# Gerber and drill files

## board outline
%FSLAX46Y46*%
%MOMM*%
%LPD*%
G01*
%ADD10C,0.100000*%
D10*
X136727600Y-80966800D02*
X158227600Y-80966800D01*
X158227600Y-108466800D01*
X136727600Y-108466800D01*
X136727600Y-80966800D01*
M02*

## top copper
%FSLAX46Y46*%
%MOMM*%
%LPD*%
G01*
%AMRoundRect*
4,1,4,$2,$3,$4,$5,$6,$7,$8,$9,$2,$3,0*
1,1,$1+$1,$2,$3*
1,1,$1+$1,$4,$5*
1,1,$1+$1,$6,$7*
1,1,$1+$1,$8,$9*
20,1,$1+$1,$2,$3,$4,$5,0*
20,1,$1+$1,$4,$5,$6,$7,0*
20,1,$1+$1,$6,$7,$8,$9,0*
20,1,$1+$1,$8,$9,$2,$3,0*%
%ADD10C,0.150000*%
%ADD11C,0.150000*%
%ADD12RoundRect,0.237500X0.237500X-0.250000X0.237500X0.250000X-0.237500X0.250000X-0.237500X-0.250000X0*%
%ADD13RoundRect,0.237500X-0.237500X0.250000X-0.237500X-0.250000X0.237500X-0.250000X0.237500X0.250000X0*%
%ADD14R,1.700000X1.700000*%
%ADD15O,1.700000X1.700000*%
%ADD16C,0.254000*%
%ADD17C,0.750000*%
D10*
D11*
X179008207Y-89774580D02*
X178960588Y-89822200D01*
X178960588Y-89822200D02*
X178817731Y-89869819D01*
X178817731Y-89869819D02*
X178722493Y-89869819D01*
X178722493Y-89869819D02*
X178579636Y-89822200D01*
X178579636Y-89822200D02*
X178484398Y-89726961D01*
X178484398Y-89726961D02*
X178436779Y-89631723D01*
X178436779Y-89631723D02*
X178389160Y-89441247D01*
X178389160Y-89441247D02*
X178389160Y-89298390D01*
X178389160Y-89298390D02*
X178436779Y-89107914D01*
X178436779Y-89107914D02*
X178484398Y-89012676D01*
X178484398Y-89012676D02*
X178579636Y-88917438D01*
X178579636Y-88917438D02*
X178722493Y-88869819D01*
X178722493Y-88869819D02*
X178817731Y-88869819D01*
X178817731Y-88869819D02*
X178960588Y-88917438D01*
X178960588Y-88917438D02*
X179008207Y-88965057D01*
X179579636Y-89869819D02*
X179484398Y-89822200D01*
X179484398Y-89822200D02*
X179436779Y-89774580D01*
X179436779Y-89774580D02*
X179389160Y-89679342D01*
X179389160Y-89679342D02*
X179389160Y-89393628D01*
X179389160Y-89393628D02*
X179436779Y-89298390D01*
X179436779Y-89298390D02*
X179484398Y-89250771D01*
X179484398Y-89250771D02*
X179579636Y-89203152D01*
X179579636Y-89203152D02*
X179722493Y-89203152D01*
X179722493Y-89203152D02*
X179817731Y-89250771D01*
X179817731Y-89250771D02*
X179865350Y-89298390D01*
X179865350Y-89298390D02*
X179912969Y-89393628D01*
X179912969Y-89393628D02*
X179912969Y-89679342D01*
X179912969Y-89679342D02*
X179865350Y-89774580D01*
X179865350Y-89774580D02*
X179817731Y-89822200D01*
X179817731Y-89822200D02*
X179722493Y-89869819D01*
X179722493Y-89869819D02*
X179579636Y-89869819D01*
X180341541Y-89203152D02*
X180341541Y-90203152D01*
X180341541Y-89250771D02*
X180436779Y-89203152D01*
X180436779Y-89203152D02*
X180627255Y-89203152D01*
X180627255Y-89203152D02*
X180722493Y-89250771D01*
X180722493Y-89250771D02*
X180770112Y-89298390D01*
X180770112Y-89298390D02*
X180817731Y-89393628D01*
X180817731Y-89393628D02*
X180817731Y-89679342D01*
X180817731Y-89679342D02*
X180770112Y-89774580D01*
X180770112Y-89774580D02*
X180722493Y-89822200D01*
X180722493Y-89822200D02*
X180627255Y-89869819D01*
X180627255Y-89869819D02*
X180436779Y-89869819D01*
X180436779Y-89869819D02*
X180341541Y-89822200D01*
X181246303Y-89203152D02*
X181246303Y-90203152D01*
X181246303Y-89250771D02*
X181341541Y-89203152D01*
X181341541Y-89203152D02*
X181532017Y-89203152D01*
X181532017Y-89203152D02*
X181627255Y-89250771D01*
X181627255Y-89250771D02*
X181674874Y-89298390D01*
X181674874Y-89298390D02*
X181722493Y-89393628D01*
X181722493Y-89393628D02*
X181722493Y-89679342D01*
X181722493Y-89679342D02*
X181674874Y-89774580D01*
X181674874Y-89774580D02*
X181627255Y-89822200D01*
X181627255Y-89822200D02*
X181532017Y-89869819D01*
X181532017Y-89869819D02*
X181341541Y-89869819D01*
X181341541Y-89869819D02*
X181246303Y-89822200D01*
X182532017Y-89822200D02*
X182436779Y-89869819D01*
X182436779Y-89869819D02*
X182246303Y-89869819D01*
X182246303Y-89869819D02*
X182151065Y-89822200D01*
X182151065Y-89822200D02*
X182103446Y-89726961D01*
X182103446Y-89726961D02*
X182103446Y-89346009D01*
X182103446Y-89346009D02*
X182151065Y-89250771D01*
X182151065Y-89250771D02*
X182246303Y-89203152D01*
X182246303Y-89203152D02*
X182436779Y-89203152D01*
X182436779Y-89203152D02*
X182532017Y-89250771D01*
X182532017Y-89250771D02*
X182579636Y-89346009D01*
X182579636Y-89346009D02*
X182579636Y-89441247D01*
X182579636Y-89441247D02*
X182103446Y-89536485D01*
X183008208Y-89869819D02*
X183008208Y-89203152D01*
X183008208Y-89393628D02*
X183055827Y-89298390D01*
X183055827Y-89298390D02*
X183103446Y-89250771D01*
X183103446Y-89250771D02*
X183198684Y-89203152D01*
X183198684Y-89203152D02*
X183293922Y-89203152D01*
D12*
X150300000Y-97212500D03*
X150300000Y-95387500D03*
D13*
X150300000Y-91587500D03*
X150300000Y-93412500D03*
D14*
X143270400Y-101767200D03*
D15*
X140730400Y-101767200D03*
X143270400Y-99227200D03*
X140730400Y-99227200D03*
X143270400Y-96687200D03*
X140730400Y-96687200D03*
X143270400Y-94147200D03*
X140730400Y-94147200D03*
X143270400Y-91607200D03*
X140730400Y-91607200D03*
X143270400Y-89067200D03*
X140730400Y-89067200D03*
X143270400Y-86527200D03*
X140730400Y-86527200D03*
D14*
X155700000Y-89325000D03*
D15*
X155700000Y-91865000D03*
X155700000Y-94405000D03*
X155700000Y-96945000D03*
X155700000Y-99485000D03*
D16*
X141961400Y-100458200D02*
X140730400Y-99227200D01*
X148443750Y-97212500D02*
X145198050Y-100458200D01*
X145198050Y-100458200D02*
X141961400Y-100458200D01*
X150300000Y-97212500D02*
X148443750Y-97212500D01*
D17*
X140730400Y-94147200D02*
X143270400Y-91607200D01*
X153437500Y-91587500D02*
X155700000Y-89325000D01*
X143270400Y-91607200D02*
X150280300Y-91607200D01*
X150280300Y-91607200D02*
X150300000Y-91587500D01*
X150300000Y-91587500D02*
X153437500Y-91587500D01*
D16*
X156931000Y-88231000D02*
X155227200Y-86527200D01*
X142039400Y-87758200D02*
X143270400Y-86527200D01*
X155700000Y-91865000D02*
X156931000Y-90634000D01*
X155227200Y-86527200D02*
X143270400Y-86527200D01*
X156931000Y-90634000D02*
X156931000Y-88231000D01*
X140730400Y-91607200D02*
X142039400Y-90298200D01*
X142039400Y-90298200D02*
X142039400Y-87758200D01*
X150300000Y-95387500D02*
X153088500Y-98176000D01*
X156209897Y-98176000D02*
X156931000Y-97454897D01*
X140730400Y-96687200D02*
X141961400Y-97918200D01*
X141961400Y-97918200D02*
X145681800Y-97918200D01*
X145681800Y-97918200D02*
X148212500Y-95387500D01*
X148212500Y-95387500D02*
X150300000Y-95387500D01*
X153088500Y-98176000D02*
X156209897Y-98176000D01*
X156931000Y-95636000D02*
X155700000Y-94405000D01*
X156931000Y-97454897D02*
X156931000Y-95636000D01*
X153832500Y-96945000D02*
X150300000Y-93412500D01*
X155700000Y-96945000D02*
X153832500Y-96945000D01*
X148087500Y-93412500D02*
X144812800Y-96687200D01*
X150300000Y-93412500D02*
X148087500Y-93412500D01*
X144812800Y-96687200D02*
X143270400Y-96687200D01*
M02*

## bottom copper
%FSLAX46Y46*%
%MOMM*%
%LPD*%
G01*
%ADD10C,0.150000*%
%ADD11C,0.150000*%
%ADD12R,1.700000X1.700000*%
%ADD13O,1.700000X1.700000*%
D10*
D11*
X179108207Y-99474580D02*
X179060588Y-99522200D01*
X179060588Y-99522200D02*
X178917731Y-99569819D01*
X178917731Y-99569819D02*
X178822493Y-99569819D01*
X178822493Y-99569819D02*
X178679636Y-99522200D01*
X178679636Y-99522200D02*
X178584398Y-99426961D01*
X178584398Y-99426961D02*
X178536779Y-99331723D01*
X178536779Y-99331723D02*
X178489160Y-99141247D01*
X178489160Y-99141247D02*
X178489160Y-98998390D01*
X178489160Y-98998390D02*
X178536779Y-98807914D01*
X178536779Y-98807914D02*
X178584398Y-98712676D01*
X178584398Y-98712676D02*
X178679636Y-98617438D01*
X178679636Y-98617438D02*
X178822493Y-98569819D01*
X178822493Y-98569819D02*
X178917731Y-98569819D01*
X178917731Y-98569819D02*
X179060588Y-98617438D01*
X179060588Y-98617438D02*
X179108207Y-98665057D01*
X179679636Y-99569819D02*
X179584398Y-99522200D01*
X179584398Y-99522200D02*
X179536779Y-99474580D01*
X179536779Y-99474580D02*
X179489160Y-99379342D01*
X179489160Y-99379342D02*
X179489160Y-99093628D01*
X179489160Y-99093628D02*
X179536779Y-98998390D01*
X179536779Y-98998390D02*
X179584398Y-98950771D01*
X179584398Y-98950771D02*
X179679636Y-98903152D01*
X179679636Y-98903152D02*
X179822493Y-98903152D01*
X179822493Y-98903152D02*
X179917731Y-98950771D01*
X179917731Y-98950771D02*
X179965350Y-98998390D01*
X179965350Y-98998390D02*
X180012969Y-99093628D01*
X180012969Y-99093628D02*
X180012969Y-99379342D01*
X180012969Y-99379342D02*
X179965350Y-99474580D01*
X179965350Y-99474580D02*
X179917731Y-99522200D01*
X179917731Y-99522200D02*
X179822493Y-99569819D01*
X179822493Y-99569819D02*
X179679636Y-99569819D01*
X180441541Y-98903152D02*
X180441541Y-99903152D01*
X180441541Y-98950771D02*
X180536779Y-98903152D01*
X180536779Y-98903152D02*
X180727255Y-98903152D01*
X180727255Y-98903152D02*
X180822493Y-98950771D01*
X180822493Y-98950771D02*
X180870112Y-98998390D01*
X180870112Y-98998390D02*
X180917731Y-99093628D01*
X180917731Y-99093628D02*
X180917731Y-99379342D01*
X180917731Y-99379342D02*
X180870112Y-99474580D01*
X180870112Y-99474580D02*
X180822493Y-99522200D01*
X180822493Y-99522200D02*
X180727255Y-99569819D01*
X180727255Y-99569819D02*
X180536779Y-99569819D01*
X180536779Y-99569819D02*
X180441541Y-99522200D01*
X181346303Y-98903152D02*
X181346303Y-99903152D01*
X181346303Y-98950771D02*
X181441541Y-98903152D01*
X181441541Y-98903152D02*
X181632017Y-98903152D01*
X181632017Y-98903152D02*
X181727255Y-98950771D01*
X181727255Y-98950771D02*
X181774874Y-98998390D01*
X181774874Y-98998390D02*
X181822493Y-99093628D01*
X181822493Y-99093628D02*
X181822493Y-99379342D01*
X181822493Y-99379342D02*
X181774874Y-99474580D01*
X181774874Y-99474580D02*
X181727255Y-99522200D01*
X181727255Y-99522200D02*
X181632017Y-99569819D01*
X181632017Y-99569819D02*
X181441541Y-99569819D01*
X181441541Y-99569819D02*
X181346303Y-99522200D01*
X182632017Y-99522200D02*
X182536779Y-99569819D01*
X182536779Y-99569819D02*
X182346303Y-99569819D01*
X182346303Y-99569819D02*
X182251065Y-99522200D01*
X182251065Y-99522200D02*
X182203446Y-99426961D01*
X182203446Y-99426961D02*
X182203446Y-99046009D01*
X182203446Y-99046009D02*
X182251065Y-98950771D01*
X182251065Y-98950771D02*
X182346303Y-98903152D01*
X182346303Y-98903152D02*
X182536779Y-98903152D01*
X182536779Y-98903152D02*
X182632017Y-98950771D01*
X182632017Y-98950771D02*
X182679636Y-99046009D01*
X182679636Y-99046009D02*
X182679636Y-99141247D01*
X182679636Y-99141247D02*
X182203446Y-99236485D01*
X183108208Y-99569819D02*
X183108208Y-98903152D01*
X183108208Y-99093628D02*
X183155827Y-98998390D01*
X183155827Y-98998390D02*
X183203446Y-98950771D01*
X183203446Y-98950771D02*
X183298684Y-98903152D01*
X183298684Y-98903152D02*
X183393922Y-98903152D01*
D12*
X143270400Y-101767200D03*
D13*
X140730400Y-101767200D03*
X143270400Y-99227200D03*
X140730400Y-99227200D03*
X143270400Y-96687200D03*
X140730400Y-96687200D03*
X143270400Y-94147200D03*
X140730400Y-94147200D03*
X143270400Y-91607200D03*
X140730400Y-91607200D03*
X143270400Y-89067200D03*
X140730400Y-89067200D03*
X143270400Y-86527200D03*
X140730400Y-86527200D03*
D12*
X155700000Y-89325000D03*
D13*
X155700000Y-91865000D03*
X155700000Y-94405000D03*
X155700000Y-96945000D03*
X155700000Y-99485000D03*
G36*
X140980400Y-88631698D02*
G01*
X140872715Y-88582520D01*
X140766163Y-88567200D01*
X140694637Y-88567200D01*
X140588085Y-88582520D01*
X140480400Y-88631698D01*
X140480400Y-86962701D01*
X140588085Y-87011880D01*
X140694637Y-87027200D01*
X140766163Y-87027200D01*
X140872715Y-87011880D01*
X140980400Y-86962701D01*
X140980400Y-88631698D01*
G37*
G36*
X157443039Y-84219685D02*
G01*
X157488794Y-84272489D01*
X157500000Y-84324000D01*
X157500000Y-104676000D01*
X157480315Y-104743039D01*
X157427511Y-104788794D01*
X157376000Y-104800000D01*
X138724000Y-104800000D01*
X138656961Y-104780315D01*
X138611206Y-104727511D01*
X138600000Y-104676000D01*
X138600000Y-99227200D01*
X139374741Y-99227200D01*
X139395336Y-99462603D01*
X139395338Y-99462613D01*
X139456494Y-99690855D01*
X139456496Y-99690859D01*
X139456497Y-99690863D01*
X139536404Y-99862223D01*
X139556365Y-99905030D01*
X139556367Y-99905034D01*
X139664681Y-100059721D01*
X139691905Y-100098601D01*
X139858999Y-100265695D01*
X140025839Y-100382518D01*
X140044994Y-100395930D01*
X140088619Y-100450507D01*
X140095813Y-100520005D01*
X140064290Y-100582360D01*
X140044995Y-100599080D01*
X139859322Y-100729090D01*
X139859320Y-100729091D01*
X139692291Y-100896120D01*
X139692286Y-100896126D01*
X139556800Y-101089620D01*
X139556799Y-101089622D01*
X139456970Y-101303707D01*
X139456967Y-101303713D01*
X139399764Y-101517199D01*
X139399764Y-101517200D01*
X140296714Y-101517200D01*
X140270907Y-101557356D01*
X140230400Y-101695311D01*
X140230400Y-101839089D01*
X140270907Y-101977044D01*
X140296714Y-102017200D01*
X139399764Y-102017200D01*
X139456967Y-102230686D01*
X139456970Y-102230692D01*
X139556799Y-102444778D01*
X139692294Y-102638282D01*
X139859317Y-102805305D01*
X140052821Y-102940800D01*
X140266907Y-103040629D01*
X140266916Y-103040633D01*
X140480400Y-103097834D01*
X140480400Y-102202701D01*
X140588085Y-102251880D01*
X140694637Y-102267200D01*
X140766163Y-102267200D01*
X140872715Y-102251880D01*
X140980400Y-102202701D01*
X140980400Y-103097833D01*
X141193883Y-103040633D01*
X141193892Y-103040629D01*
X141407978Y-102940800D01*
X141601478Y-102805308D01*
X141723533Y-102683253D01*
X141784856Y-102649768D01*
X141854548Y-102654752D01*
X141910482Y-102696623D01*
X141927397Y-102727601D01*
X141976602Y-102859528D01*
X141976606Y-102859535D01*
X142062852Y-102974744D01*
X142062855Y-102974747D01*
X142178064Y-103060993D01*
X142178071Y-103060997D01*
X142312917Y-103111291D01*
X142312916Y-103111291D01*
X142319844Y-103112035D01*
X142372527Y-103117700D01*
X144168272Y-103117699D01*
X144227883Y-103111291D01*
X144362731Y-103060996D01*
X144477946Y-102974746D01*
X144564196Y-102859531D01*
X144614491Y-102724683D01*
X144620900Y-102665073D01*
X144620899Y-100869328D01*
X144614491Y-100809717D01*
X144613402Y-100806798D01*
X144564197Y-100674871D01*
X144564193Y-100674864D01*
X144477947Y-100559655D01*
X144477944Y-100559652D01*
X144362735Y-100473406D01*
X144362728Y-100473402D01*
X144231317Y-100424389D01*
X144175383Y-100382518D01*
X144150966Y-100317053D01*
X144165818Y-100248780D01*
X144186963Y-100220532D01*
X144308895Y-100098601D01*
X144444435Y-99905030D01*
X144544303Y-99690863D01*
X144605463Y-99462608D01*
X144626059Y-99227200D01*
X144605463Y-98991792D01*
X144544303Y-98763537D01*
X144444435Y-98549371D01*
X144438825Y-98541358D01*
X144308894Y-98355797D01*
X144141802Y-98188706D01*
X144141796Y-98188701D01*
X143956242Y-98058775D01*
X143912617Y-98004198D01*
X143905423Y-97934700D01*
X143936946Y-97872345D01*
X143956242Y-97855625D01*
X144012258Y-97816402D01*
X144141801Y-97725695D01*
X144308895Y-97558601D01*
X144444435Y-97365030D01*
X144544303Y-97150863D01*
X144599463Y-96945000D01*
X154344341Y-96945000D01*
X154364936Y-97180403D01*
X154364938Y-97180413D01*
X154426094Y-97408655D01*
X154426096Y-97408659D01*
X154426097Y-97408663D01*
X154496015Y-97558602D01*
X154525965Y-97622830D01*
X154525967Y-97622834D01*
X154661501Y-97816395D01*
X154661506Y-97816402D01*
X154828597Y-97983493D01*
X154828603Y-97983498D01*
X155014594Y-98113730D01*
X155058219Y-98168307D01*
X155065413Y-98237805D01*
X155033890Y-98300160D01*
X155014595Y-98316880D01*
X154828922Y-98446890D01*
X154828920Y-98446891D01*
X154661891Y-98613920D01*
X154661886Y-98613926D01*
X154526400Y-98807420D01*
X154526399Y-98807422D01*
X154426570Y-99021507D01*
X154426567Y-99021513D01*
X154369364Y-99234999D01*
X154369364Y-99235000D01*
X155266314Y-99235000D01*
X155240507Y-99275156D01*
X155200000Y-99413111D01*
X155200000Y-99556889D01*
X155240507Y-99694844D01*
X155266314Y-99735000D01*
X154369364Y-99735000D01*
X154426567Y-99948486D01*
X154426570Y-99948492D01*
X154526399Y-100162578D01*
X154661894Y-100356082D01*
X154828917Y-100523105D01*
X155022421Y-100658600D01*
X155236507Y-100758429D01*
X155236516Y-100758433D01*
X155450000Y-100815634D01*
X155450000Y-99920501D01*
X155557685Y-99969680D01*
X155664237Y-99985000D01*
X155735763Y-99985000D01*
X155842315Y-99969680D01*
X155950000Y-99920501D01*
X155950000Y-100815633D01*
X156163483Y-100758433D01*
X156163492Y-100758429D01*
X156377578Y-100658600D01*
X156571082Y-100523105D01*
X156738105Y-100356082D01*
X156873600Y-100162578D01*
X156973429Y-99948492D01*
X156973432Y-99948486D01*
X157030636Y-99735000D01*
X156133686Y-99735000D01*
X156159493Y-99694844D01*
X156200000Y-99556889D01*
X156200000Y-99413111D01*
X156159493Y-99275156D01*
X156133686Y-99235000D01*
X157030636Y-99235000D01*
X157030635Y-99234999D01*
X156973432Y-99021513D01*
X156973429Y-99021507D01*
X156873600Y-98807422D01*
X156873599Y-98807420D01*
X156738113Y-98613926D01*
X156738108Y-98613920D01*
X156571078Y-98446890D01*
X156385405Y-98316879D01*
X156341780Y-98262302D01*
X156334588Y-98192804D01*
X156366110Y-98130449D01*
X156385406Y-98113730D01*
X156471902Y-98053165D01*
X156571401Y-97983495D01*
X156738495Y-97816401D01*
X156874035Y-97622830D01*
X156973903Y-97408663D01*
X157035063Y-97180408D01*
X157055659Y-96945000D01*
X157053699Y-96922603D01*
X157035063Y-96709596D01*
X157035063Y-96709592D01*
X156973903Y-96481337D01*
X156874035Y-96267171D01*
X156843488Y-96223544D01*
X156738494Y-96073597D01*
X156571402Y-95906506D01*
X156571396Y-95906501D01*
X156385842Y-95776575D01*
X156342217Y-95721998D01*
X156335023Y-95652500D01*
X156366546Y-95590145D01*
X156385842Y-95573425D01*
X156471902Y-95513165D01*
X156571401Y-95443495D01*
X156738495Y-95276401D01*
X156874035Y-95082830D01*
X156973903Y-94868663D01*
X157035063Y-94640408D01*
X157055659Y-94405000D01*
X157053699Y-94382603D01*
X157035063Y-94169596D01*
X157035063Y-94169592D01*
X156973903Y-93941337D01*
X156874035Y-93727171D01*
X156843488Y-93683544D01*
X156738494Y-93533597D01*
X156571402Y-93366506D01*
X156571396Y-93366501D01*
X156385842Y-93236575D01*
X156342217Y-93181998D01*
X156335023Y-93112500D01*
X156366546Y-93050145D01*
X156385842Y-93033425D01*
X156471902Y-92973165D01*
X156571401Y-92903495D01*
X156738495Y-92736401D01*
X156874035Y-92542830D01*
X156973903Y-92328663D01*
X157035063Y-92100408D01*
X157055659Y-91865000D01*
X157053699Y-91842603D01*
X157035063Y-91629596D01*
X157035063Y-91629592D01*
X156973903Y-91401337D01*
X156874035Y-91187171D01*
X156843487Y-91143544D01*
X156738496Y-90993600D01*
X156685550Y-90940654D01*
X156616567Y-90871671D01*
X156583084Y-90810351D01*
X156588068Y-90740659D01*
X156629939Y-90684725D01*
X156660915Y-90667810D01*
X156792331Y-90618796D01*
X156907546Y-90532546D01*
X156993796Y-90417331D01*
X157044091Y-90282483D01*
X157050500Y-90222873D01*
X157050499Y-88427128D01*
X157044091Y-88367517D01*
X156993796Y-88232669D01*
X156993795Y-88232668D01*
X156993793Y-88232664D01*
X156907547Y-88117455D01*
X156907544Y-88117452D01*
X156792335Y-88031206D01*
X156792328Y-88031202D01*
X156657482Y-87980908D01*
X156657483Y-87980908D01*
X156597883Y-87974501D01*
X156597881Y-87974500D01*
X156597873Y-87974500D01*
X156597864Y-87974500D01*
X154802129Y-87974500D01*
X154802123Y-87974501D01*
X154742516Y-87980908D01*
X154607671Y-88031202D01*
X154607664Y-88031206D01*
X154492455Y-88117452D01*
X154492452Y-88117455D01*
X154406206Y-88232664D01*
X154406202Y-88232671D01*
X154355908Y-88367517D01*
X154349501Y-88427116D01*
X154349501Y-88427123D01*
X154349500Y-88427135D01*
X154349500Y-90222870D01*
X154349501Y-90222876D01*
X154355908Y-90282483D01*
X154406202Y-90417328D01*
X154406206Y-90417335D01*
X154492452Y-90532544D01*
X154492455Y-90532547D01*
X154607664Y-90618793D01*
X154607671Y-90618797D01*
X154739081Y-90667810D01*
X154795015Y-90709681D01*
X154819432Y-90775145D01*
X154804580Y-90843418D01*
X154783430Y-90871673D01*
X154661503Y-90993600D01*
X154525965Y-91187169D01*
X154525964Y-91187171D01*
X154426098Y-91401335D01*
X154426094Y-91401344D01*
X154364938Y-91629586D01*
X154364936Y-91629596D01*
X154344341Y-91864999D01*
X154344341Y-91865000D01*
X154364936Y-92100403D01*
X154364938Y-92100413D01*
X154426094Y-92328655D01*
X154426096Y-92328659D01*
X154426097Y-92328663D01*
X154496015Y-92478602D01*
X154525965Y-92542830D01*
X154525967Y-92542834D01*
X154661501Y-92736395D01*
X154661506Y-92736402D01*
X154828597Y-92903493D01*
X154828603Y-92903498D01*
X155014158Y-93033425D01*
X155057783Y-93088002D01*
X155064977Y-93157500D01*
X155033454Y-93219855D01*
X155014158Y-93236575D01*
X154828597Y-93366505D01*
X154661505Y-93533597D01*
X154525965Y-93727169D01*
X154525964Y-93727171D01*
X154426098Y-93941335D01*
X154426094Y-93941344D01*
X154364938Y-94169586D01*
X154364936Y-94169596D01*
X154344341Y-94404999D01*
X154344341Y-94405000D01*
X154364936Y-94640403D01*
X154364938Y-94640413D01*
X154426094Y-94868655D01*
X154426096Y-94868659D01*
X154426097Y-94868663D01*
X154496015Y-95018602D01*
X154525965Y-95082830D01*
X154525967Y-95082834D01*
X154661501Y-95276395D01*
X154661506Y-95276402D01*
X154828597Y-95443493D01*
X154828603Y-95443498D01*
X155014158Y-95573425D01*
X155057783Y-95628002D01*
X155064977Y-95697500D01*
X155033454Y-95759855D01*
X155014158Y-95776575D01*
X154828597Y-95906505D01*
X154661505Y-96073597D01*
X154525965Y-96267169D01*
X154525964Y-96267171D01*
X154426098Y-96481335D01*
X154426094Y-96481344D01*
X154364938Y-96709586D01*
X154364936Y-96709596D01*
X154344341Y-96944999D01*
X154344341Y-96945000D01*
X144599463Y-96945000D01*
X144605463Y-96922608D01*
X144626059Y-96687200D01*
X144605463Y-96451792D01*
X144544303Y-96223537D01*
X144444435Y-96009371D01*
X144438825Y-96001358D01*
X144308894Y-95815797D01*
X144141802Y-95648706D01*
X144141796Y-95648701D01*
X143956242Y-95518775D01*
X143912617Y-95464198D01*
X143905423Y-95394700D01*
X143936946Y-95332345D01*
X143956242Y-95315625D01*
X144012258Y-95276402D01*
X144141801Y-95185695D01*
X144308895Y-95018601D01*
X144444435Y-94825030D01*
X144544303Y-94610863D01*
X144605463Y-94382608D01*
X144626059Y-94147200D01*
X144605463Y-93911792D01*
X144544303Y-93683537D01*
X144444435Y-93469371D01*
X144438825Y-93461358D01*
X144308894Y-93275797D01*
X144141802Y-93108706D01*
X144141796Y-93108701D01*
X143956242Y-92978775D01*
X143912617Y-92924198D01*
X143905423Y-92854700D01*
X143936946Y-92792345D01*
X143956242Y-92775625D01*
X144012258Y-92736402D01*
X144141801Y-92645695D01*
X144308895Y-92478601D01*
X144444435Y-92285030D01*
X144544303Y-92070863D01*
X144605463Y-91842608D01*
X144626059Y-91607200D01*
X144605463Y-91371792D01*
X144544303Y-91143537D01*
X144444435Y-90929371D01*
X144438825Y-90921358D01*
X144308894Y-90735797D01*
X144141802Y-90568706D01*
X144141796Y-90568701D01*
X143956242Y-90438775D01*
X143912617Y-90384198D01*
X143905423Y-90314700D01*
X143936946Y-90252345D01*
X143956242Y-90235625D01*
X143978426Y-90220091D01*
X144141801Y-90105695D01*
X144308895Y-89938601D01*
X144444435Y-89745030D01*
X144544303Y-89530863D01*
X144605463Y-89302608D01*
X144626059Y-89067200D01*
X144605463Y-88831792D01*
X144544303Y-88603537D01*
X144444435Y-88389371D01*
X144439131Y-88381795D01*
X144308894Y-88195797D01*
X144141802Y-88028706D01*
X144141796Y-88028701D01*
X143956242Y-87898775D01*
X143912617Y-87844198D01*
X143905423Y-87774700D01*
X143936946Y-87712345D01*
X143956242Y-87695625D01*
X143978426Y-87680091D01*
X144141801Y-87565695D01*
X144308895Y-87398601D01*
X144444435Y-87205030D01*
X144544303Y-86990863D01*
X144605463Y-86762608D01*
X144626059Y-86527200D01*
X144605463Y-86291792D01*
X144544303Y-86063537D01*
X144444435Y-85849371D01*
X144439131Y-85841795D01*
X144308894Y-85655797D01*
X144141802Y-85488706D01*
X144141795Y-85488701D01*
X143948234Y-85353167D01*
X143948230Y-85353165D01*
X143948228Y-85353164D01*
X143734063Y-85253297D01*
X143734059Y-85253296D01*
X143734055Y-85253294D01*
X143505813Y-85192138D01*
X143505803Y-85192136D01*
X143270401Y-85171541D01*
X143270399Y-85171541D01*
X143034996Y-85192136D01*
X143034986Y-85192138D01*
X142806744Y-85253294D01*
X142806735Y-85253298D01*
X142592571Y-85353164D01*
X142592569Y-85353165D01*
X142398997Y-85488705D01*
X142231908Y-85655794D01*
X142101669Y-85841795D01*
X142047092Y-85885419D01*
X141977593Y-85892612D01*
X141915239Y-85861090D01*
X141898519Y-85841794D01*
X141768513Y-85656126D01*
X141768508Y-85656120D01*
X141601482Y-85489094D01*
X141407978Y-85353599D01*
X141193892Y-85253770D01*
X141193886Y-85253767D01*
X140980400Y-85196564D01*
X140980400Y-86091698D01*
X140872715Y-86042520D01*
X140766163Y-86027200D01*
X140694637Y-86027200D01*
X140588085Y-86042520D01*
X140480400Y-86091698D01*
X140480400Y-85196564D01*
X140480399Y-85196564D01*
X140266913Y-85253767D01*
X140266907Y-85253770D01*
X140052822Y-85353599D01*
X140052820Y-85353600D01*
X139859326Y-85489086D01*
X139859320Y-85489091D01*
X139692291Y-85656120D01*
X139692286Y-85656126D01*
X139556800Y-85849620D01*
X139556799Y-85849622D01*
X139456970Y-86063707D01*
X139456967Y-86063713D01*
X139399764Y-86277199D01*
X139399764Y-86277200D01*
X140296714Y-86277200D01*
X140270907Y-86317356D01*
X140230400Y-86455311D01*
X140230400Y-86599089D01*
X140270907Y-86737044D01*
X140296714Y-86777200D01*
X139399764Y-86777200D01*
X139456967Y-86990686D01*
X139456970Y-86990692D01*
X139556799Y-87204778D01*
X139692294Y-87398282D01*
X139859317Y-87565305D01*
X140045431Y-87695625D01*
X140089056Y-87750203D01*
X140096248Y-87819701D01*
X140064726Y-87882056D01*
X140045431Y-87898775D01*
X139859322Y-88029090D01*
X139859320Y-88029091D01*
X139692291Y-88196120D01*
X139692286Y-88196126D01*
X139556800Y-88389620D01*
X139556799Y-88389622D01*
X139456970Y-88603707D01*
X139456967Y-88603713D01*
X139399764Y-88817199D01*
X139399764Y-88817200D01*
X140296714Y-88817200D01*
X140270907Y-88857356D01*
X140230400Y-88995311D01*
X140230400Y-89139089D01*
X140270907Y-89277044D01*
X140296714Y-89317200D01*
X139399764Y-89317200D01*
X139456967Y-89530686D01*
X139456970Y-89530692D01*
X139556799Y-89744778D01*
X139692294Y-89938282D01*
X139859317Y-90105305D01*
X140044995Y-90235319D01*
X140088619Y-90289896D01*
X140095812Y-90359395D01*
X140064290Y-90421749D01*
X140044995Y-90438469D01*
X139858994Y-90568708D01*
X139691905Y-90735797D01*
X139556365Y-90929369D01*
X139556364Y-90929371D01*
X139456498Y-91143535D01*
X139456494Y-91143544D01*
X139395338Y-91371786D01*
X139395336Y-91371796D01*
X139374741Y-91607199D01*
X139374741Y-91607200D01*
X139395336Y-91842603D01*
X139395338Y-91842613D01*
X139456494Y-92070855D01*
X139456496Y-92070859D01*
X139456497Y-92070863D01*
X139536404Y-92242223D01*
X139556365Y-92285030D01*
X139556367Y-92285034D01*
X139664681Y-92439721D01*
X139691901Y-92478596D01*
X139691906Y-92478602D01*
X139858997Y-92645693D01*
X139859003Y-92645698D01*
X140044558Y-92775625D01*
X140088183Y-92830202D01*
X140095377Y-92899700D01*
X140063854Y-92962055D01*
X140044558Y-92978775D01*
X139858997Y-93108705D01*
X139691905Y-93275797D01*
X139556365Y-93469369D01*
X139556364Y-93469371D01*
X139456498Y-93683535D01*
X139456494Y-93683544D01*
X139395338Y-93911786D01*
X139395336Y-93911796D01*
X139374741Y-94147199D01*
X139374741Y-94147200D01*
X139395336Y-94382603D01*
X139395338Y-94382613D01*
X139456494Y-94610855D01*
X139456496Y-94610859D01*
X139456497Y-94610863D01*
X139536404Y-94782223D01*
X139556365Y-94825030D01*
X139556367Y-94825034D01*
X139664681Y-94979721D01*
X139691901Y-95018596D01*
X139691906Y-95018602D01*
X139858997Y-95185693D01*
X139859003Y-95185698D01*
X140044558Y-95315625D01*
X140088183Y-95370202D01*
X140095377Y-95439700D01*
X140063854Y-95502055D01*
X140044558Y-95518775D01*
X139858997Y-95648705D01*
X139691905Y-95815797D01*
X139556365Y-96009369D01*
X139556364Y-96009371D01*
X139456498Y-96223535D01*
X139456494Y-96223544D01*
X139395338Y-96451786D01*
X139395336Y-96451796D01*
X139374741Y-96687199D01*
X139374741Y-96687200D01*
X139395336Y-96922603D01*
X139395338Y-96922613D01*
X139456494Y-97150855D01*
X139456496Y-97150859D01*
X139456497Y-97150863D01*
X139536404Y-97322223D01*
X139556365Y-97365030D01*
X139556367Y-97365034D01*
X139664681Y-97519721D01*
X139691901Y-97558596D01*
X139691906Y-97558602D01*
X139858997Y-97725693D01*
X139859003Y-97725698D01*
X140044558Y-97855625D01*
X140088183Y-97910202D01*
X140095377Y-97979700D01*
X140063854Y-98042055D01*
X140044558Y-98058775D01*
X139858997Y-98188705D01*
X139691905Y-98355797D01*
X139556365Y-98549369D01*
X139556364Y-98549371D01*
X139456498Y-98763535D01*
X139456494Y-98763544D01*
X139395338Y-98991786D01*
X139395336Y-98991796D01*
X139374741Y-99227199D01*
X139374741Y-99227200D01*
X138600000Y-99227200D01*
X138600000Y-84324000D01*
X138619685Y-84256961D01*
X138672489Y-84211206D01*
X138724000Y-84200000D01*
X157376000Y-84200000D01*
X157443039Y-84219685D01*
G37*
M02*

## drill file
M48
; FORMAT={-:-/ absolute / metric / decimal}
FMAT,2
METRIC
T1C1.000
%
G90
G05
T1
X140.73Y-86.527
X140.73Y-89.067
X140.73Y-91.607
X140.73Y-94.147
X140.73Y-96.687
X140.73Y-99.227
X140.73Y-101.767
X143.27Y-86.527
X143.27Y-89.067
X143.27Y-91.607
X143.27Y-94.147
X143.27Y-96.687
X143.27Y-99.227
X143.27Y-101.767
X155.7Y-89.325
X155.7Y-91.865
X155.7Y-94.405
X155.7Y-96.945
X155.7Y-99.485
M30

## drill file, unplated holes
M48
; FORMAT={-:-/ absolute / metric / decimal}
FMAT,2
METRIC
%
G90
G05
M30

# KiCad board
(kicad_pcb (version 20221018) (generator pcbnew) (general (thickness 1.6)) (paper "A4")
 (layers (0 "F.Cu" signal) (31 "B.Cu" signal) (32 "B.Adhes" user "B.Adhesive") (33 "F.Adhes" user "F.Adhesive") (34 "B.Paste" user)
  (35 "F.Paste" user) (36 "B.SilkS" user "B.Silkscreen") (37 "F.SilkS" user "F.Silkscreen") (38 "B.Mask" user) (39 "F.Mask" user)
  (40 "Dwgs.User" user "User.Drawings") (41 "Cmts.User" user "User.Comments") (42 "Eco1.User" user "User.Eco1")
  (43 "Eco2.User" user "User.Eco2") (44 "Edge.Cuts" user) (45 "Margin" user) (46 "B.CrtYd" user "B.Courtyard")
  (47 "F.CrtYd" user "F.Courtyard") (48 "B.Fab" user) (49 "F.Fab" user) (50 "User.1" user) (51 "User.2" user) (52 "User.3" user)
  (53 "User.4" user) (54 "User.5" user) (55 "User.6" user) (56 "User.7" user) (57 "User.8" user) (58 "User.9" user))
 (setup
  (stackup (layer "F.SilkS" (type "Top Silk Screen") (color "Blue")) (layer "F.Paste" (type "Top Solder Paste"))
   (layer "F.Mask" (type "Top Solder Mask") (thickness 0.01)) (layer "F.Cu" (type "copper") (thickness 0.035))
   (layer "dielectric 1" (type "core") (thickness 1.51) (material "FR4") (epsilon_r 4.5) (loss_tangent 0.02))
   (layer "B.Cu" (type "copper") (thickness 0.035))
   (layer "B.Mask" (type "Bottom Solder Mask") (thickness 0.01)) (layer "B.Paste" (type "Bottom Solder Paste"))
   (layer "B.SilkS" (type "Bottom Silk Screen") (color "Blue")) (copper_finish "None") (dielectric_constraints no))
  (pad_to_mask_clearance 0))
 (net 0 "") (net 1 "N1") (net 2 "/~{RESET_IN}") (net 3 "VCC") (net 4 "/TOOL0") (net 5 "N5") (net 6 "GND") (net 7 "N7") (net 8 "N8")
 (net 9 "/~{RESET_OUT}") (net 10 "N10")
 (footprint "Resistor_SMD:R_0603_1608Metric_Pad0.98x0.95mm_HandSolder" (layer "F.Cu") (at 150.3 96.3 90)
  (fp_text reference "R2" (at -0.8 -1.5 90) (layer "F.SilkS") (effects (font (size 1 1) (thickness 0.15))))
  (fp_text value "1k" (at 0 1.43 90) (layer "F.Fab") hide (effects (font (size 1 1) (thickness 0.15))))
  (pad "1" smd roundrect (at -0.9125 0 90) (size 0.975 0.95) (layers "F.Cu" "F.Paste" "F.Mask") (roundrect_rratio 0.25) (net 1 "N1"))
  (pad "2" smd roundrect (at 0.9125 0 90) (size 0.975 0.95) (layers "F.Cu" "F.Paste" "F.Mask") (roundrect_rratio 0.25)
   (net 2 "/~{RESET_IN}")))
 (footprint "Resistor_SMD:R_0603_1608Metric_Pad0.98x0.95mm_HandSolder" (layer "F.Cu") (at 150.3 92.5 -90)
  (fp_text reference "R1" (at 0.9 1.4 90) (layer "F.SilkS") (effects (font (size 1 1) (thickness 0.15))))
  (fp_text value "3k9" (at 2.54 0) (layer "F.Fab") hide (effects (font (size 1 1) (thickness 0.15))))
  (pad "1" smd roundrect (at -0.9125 0 270) (size 0.975 0.95) (layers "F.Cu" "F.Paste" "F.Mask") (roundrect_rratio 0.25) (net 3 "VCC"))
  (pad "2" smd roundrect (at 0.9125 0 270) (size 0.975 0.95) (layers "F.Cu" "F.Paste" "F.Mask") (roundrect_rratio 0.25) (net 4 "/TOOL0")))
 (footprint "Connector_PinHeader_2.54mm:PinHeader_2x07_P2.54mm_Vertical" (layer "F.Cu") (at 143.2704 101.7672 180)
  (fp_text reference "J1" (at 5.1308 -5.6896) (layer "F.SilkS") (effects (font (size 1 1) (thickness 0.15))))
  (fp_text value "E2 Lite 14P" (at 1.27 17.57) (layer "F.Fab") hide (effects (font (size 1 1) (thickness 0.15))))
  (pad "1" thru_hole rect (at 0 0 180) (size 1.7 1.7) (drill 1) (layers "*.Cu" "*.Mask") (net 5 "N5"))
  (pad "2" thru_hole oval (at 2.54 0 180) (size 1.7 1.7) (drill 1) (layers "*.Cu" "*.Mask") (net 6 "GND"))
  (pad "3" thru_hole oval (at 0 2.54 180) (size 1.7 1.7) (drill 1) (layers "*.Cu" "*.Mask") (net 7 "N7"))
  (pad "4" thru_hole oval (at 2.54 2.54 180) (size 1.7 1.7) (drill 1) (layers "*.Cu" "*.Mask") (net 1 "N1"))
  (pad "5" thru_hole oval (at 0 5.08 180) (size 1.7 1.7) (drill 1) (layers "*.Cu" "*.Mask") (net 4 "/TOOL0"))
  (pad "6" thru_hole oval (at 2.54 5.08 180) (size 1.7 1.7) (drill 1) (layers "*.Cu" "*.Mask") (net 2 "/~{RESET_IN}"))
  (pad "7" thru_hole oval (at 0 7.62 180) (size 1.7 1.7) (drill 1) (layers "*.Cu" "*.Mask") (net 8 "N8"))
  (pad "8" thru_hole oval (at 2.54 7.62 180) (size 1.7 1.7) (drill 1) (layers "*.Cu" "*.Mask") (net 3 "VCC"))
  (pad "9" thru_hole oval (at 0 10.16 180) (size 1.7 1.7) (drill 1) (layers "*.Cu" "*.Mask") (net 3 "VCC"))
  (pad "10" thru_hole oval (at 2.54 10.16 180) (size 1.7 1.7) (drill 1) (layers "*.Cu" "*.Mask") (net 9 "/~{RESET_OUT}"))
  (pad "11" thru_hole oval (at 0 12.7 180) (size 1.7 1.7) (drill 1) (layers "*.Cu" "*.Mask") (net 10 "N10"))
  (pad "12" thru_hole oval (at 2.54 12.7 180) (size 1.7 1.7) (drill 1) (layers "*.Cu" "*.Mask") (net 6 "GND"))
  (pad "13" thru_hole oval (at 0 15.24 180) (size 1.7 1.7) (drill 1) (layers "*.Cu" "*.Mask") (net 9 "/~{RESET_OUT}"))
  (pad "14" thru_hole oval (at 2.54 15.24 180) (size 1.7 1.7) (drill 1) (layers "*.Cu" "*.Mask") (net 6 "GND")))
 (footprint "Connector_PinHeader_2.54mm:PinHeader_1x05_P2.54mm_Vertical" (layer "B.Cu") (at 155.7 89.325 180)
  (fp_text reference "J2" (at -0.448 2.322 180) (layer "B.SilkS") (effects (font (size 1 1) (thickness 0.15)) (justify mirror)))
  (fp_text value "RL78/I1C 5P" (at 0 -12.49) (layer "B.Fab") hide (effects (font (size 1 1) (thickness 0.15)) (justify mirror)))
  (pad "1" thru_hole rect (at 0 0 180) (size 1.7 1.7) (drill 1) (layers "*.Cu" "*.Mask") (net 3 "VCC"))
  (pad "2" thru_hole oval (at 0 -2.54 180) (size 1.7 1.7) (drill 1) (layers "*.Cu" "*.Mask") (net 9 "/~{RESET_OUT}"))
  (pad "3" thru_hole oval (at 0 -5.08 180) (size 1.7 1.7) (drill 1) (layers "*.Cu" "*.Mask") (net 2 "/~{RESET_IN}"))
  (pad "4" thru_hole oval (at 0 -7.62 180) (size 1.7 1.7) (drill 1) (layers "*.Cu" "*.Mask") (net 4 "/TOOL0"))
  (pad "5" thru_hole oval (at 0 -10.16 180) (size 1.7 1.7) (drill 1) (layers "*.Cu" "*.Mask") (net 6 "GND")))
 (gr_rect (start 136.7276 80.9668) (end 158.2276 108.4668) (stroke (width 0.1) (type default)) (fill none) (layer "Edge.Cuts"))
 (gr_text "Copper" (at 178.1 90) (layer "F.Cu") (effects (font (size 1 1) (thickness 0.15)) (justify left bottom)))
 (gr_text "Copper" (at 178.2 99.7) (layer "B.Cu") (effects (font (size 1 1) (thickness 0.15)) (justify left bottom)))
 (segment (start 141.9614 100.4582) (end 140.7304 99.2272) (width 0.254) (layer "F.Cu") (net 1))
 (segment (start 148.44375 97.2125) (end 145.19805 100.4582) (width 0.254) (layer "F.Cu") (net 1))
 (segment (start 145.19805 100.4582) (end 141.9614 100.4582) (width 0.254) (layer "F.Cu") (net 1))
 (segment (start 150.3 97.2125) (end 148.44375 97.2125) (width 0.254) (layer "F.Cu") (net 1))
 (segment (start 140.7304 94.1472) (end 143.2704 91.6072) (width 0.75) (layer "F.Cu") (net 3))
 (segment (start 153.4375 91.5875) (end 155.7 89.325) (width 0.75) (layer "F.Cu") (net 3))
 (segment (start 143.2704 91.6072) (end 150.2803 91.6072) (width 0.75) (layer "F.Cu") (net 3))
 (segment (start 150.2803 91.6072) (end 150.3 91.5875) (width 0.75) (layer "F.Cu") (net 3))
 (segment (start 150.3 91.5875) (end 153.4375 91.5875) (width 0.75) (layer "F.Cu") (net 3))
 (segment (start 156.931 88.231) (end 155.2272 86.5272) (width 0.254) (layer "F.Cu") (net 9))
 (segment (start 142.0394 87.7582) (end 143.2704 86.5272) (width 0.254) (layer "F.Cu") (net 9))
 (segment (start 155.7 91.865) (end 156.931 90.634) (width 0.254) (layer "F.Cu") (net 9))
 (segment (start 155.2272 86.5272) (end 143.2704 86.5272) (width 0.254) (layer "F.Cu") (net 9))
 (segment (start 156.931 90.634) (end 156.931 88.231) (width 0.254) (layer "F.Cu") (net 9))
 (segment (start 140.7304 91.6072) (end 142.0394 90.2982) (width 0.254) (layer "F.Cu") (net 9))
 (segment (start 142.0394 90.2982) (end 142.0394 87.7582) (width 0.254) (layer "F.Cu") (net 9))
 (segment (start 150.3 95.3875) (end 153.0885 98.176) (width 0.254) (layer "F.Cu") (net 2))
 (segment (start 156.209897 98.176) (end 156.931 97.454897) (width 0.254) (layer "F.Cu") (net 2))
 (segment (start 140.7304 96.6872) (end 141.9614 97.9182) (width 0.254) (layer "F.Cu") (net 2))
 (segment (start 141.9614 97.9182) (end 145.6818 97.9182) (width 0.254) (layer "F.Cu") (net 2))
 (segment (start 145.6818 97.9182) (end 148.2125 95.3875) (width 0.254) (layer "F.Cu") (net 2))
 (segment (start 148.2125 95.3875) (end 150.3 95.3875) (width 0.254) (layer "F.Cu") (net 2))
 (segment (start 153.0885 98.176) (end 156.209897 98.176) (width 0.254) (layer "F.Cu") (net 2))
 (segment (start 156.931 95.636) (end 155.7 94.405) (width 0.254) (layer "F.Cu") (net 2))
 (segment (start 156.931 97.454897) (end 156.931 95.636) (width 0.254) (layer "F.Cu") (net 2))
 (segment (start 153.8325 96.945) (end 150.3 93.4125) (width 0.254) (layer "F.Cu") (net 4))
 (segment (start 155.7 96.945) (end 153.8325 96.945) (width 0.254) (layer "F.Cu") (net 4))
 (segment (start 148.0875 93.4125) (end 144.8128 96.6872) (width 0.254) (layer "F.Cu") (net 4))
 (segment (start 150.3 93.4125) (end 148.0875 93.4125) (width 0.254) (layer "F.Cu") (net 4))
 (segment (start 144.8128 96.6872) (end 143.2704 96.6872) (width 0.254) (layer "F.Cu") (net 4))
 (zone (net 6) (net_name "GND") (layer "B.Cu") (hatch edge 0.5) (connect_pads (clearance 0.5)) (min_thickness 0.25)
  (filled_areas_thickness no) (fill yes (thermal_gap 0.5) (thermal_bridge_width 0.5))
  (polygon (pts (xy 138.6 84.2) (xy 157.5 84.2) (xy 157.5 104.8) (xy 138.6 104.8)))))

